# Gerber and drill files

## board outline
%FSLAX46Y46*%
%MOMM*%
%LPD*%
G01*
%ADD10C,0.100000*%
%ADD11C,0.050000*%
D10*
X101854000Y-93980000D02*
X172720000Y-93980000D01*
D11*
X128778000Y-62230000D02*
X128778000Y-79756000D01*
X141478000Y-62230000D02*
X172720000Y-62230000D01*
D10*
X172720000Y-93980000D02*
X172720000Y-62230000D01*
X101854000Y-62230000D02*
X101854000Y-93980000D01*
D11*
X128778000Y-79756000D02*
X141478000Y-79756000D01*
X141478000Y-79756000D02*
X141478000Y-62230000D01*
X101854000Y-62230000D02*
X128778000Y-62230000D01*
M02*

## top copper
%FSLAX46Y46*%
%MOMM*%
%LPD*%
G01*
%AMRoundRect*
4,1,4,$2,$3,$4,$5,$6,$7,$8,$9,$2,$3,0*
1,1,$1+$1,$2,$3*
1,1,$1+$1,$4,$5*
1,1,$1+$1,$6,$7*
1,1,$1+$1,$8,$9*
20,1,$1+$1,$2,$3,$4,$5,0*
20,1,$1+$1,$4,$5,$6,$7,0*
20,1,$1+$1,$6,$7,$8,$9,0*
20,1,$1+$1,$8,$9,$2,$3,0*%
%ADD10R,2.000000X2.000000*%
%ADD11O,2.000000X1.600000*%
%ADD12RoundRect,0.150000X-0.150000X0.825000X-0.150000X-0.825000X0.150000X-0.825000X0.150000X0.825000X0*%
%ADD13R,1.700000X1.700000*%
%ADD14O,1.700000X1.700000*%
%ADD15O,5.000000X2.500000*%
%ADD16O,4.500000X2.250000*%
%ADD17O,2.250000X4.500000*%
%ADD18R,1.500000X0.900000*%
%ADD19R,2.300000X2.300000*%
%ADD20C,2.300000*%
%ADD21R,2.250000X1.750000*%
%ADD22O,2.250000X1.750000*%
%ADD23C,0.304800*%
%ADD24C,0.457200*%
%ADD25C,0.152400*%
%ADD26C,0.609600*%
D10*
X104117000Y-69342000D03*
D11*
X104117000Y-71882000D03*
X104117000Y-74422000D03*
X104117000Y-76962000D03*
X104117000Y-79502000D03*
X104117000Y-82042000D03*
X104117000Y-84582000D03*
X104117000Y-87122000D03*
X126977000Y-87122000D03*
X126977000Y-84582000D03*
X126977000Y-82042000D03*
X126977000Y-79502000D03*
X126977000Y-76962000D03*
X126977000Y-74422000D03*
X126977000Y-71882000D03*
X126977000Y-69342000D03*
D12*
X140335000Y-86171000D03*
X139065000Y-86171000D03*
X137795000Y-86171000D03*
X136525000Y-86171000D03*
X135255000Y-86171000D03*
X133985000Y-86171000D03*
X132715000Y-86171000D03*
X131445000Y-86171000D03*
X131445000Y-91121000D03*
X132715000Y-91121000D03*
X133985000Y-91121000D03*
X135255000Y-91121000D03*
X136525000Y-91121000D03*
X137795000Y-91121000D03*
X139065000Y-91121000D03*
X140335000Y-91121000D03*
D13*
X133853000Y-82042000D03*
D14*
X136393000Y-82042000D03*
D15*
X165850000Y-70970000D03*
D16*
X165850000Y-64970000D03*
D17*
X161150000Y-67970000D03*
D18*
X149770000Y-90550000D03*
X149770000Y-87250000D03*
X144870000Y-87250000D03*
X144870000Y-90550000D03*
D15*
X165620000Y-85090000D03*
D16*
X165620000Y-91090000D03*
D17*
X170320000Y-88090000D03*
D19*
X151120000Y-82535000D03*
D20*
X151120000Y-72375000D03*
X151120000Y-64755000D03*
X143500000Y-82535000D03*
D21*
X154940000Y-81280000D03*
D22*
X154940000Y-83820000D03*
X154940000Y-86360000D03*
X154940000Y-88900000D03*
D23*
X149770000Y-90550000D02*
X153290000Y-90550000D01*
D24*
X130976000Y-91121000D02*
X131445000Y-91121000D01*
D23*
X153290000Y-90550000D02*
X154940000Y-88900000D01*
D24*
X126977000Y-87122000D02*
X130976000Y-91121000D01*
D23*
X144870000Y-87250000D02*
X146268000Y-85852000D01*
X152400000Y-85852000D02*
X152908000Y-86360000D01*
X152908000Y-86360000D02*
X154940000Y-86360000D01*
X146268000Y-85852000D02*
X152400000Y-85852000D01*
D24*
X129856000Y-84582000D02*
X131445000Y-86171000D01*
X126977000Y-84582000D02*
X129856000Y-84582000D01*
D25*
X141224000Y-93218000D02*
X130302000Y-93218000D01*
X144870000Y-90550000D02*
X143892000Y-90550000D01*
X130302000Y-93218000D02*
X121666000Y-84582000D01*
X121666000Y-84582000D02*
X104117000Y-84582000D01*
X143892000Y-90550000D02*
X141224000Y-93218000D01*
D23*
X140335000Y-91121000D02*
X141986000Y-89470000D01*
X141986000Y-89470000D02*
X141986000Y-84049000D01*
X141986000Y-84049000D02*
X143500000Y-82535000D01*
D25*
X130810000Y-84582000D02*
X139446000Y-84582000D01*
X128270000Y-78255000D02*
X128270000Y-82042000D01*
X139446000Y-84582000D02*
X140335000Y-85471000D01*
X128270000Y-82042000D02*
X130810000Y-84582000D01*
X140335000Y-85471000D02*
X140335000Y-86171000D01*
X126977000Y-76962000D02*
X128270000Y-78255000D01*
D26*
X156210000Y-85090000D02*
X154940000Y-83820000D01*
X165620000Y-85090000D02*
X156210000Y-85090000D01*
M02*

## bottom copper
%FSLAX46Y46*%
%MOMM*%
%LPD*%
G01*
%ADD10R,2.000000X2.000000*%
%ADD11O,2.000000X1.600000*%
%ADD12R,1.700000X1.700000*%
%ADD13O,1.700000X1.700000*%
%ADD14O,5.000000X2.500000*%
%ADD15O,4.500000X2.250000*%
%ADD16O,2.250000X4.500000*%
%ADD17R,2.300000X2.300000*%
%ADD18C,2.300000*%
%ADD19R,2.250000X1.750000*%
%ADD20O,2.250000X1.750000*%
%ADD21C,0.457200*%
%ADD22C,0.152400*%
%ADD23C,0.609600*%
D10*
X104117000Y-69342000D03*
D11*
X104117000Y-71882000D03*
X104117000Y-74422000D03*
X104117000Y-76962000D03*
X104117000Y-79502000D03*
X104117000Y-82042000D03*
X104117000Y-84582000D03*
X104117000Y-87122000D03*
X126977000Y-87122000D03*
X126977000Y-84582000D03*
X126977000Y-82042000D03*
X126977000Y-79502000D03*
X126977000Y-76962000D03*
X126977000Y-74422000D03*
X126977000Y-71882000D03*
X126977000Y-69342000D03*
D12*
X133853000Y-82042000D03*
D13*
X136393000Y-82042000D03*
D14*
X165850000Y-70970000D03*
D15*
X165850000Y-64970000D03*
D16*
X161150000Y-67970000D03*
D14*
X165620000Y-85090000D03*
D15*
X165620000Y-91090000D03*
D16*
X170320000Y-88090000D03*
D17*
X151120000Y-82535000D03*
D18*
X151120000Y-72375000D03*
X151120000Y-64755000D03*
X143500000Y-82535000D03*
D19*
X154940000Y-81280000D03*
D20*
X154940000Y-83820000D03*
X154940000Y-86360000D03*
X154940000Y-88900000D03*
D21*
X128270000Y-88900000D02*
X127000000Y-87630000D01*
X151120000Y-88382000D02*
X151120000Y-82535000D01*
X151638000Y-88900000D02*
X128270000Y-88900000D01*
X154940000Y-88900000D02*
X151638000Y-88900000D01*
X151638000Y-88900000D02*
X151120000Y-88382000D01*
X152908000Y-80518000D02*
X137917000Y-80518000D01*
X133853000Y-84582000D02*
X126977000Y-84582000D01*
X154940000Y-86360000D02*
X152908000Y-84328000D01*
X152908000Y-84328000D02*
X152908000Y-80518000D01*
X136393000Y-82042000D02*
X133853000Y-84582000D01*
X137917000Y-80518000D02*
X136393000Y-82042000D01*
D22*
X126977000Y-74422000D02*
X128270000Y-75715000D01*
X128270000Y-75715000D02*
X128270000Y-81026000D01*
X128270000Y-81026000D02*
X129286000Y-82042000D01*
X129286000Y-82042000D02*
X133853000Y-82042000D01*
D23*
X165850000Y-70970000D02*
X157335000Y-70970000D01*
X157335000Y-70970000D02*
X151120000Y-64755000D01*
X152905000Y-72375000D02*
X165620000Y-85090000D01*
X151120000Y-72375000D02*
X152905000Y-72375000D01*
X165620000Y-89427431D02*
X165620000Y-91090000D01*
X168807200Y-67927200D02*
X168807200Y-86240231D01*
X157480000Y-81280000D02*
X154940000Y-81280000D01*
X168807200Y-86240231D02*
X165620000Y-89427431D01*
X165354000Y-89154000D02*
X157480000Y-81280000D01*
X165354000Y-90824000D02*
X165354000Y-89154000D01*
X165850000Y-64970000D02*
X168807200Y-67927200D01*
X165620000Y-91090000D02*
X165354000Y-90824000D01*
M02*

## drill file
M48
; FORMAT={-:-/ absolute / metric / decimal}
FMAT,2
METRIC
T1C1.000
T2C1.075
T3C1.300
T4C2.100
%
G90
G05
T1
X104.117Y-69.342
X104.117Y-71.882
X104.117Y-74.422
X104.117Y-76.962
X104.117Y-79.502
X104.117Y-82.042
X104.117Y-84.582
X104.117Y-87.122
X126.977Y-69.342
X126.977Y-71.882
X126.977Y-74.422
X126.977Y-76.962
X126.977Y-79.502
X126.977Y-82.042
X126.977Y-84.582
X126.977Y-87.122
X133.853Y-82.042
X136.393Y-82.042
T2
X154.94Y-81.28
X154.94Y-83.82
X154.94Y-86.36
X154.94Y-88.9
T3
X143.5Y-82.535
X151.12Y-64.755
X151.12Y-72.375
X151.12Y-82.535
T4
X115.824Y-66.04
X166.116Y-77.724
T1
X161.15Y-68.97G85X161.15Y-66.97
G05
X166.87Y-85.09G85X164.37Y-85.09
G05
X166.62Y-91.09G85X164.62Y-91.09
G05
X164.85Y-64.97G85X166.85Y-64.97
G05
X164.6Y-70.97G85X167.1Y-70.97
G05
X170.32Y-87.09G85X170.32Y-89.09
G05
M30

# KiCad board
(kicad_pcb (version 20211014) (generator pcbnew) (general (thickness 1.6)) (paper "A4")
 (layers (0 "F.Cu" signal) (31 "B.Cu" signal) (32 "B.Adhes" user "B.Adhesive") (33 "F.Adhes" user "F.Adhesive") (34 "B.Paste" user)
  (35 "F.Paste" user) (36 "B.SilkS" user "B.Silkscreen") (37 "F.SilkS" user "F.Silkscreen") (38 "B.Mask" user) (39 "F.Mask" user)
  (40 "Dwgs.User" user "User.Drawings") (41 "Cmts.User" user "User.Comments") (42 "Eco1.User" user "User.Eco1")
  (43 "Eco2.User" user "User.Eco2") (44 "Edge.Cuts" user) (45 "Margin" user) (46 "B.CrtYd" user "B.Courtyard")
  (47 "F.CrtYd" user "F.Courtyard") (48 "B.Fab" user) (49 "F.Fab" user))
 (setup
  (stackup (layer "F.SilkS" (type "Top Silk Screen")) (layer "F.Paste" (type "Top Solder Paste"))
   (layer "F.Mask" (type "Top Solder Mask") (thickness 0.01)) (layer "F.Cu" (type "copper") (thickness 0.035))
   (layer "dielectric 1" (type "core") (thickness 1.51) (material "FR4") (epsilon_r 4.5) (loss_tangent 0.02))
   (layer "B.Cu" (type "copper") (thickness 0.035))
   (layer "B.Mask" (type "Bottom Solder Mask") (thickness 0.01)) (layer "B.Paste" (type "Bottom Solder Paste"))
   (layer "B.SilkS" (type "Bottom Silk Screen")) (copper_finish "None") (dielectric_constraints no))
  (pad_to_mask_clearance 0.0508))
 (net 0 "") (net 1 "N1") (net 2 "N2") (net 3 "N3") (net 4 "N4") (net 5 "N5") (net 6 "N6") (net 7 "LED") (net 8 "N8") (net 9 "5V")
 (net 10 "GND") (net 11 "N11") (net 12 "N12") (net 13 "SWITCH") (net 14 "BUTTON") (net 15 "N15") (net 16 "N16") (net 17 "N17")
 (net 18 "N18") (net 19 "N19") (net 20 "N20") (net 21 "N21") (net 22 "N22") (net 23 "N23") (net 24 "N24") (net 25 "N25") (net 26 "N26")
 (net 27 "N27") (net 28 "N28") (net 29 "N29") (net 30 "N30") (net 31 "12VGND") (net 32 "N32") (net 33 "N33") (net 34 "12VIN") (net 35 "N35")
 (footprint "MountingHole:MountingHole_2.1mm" (layer "F.Cu") (at 115.824 66.04)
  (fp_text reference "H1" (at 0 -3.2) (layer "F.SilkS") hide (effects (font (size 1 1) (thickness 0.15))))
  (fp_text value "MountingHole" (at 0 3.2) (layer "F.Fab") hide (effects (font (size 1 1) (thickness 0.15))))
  (pad "" np_thru_hole circle (at 0 0) (size 2.1 2.1) (drill 2.1) (layers *.Cu *.Mask)))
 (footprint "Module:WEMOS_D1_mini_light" (layer "F.Cu") (at 104.117 69.342)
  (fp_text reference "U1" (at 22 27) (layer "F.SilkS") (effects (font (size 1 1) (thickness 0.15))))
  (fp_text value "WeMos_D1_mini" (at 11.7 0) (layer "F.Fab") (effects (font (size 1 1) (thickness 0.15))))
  (pad "1" thru_hole rect (at 0 0) (size 2 2) (drill 1) (layers *.Cu *.Mask) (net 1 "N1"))
  (pad "2" thru_hole oval (at 0 2.54) (size 2 1.6) (drill 1) (layers *.Cu *.Mask) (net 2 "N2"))
  (pad "3" thru_hole oval (at 0 5.08) (size 2 1.6) (drill 1) (layers *.Cu *.Mask) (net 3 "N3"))
  (pad "4" thru_hole oval (at 0 7.62) (size 2 1.6) (drill 1) (layers *.Cu *.Mask) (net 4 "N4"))
  (pad "5" thru_hole oval (at 0 10.16) (size 2 1.6) (drill 1) (layers *.Cu *.Mask) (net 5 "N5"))
  (pad "6" thru_hole oval (at 0 12.7) (size 2 1.6) (drill 1) (layers *.Cu *.Mask) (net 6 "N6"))
  (pad "7" thru_hole oval (at 0 15.24) (size 2 1.6) (drill 1) (layers *.Cu *.Mask) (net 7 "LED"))
  (pad "8" thru_hole oval (at 0 17.78) (size 2 1.6) (drill 1) (layers *.Cu *.Mask) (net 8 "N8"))
  (pad "9" thru_hole oval (at 22.86 17.78) (size 2 1.6) (drill 1) (layers *.Cu *.Mask) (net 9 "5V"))
  (pad "10" thru_hole oval (at 22.86 15.24) (size 2 1.6) (drill 1) (layers *.Cu *.Mask) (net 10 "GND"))
  (pad "11" thru_hole oval (at 22.86 12.7) (size 2 1.6) (drill 1) (layers *.Cu *.Mask) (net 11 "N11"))
  (pad "12" thru_hole oval (at 22.86 10.16) (size 2 1.6) (drill 1) (layers *.Cu *.Mask) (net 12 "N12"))
  (pad "13" thru_hole oval (at 22.86 7.62) (size 2 1.6) (drill 1) (layers *.Cu *.Mask) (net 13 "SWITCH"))
  (pad "14" thru_hole oval (at 22.86 5.08) (size 2 1.6) (drill 1) (layers *.Cu *.Mask) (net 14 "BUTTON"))
  (pad "15" thru_hole oval (at 22.86 2.54) (size 2 1.6) (drill 1) (layers *.Cu *.Mask) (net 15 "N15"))
  (pad "16" thru_hole oval (at 22.86 0) (size 2 1.6) (drill 1) (layers *.Cu *.Mask) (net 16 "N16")))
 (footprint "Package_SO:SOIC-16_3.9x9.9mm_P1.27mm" (layer "F.Cu") (at 135.89 88.646 -90)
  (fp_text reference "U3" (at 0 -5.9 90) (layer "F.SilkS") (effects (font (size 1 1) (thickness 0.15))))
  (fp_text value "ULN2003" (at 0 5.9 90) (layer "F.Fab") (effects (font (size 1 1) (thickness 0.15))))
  (pad "1" smd roundrect (at -2.475 -4.445 270) (size 1.95 0.6) (layers "F.Cu" "F.Paste" "F.Mask") (roundrect_rratio 0.25) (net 13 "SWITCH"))
  (pad "2" smd roundrect (at -2.475 -3.175 270) (size 1.95 0.6) (layers "F.Cu" "F.Paste" "F.Mask") (roundrect_rratio 0.25) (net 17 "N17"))
  (pad "3" smd roundrect (at -2.475 -1.905 270) (size 1.95 0.6) (layers "F.Cu" "F.Paste" "F.Mask") (roundrect_rratio 0.25) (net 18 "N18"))
  (pad "4" smd roundrect (at -2.475 -0.635 270) (size 1.95 0.6) (layers "F.Cu" "F.Paste" "F.Mask") (roundrect_rratio 0.25) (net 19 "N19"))
  (pad "5" smd roundrect (at -2.475 0.635 270) (size 1.95 0.6) (layers "F.Cu" "F.Paste" "F.Mask") (roundrect_rratio 0.25) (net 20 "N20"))
  (pad "6" smd roundrect (at -2.475 1.905 270) (size 1.95 0.6) (layers "F.Cu" "F.Paste" "F.Mask") (roundrect_rratio 0.25) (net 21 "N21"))
  (pad "7" smd roundrect (at -2.475 3.175 270) (size 1.95 0.6) (layers "F.Cu" "F.Paste" "F.Mask") (roundrect_rratio 0.25) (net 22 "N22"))
  (pad "8" smd roundrect (at -2.475 4.445 270) (size 1.95 0.6) (layers "F.Cu" "F.Paste" "F.Mask") (roundrect_rratio 0.25) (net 10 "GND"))
  (pad "9" smd roundrect (at 2.475 4.445 270) (size 1.95 0.6) (layers "F.Cu" "F.Paste" "F.Mask") (roundrect_rratio 0.25) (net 9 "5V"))
  (pad "10" smd roundrect (at 2.475 3.175 270) (size 1.95 0.6) (layers "F.Cu" "F.Paste" "F.Mask") (roundrect_rratio 0.25) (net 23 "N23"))
  (pad "11" smd roundrect (at 2.475 1.905 270) (size 1.95 0.6) (layers "F.Cu" "F.Paste" "F.Mask") (roundrect_rratio 0.25) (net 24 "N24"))
  (pad "12" smd roundrect (at 2.475 0.635 270) (size 1.95 0.6) (layers "F.Cu" "F.Paste" "F.Mask") (roundrect_rratio 0.25) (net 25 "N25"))
  (pad "13" smd roundrect (at 2.475 -0.635 270) (size 1.95 0.6) (layers "F.Cu" "F.Paste" "F.Mask") (roundrect_rratio 0.25) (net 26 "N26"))
  (pad "14" smd roundrect (at 2.475 -1.905 270) (size 1.95 0.6) (layers "F.Cu" "F.Paste" "F.Mask") (roundrect_rratio 0.25) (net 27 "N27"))
  (pad "15" smd roundrect (at 2.475 -3.175 270) (size 1.95 0.6) (layers "F.Cu" "F.Paste" "F.Mask") (roundrect_rratio 0.25) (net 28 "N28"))
  (pad "16" smd roundrect (at 2.475 -4.445 270) (size 1.95 0.6) (layers "F.Cu" "F.Paste" "F.Mask") (roundrect_rratio 0.25) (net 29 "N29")))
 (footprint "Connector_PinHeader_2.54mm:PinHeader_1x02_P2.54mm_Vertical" (layer "F.Cu") (at 133.853 82.042 90)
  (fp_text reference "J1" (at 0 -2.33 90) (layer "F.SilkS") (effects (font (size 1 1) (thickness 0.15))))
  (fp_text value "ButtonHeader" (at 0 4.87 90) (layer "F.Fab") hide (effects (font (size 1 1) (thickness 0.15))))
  (pad "1" thru_hole rect (at 0 0 90) (size 1.7 1.7) (drill 1) (layers *.Cu *.Mask) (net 14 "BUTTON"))
  (pad "2" thru_hole oval (at 0 2.54 90) (size 1.7 1.7) (drill 1) (layers *.Cu *.Mask) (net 10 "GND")))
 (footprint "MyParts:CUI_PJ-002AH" (layer "F.Cu") (at 165.85 70.97 90)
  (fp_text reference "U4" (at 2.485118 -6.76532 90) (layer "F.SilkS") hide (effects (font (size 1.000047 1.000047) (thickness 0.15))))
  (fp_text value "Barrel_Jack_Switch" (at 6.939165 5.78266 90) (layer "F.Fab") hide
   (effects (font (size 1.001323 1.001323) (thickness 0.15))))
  (pad "1" thru_hole oval locked (at 0 0 90) (size 2.5 5) (drill oval 1 3.5) (layers *.Cu *.Mask) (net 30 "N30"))
  (pad "2" thru_hole oval locked (at 6 0 90) (size 2.25 4.5) (drill oval 1 3) (layers *.Cu *.Mask) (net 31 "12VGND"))
  (pad "3" thru_hole oval locked (at 3 -4.7 90) (size 4.5 2.25) (drill oval 3 1) (layers *.Cu *.Mask) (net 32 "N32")))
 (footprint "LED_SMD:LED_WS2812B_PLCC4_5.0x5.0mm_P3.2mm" (layer "F.Cu") (at 147.32 88.9 180)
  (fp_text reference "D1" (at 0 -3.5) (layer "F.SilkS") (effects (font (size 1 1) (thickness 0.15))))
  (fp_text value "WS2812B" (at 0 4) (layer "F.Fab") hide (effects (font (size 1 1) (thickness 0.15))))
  (pad "1" smd rect (at -2.45 -1.65 180) (size 1.5 0.9) (layers "F.Cu" "F.Paste" "F.Mask") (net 9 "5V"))
  (pad "2" smd rect (at -2.45 1.65 180) (size 1.5 0.9) (layers "F.Cu" "F.Paste" "F.Mask") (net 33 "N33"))
  (pad "3" smd rect (at 2.45 1.65 180) (size 1.5 0.9) (layers "F.Cu" "F.Paste" "F.Mask") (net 10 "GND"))
  (pad "4" smd rect (at 2.45 -1.65 180) (size 1.5 0.9) (layers "F.Cu" "F.Paste" "F.Mask") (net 7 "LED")))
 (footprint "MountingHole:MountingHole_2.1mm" (layer "F.Cu") (at 166.116 77.724)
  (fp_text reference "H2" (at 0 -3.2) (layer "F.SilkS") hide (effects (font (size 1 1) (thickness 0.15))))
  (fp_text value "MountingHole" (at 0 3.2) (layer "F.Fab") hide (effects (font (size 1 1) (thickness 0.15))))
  (pad "" np_thru_hole circle (at 0 0) (size 2.1 2.1) (drill 2.1) (layers *.Cu *.Mask)))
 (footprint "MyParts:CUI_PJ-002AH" (layer "F.Cu") (at 165.62 85.09 -90)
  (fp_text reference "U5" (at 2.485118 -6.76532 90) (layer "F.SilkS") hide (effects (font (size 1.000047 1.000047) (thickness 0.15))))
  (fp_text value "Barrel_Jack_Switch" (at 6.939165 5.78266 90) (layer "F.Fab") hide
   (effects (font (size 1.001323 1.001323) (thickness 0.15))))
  (pad "1" thru_hole oval locked (at 0 0 270) (size 2.5 5) (drill oval 1 3.5) (layers *.Cu *.Mask) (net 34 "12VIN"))
  (pad "2" thru_hole oval locked (at 6 0 270) (size 2.25 4.5) (drill oval 1 3) (layers *.Cu *.Mask) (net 31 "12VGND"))
  (pad "3" thru_hole oval locked (at 3 -4.7 270) (size 4.5 2.25) (drill oval 3 1) (layers *.Cu *.Mask) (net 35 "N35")))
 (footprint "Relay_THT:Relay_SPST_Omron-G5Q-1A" (layer "F.Cu") (at 151.12 82.535 90)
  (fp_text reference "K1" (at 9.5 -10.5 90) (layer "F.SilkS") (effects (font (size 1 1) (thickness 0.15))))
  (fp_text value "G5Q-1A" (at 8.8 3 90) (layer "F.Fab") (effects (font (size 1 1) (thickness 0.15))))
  (pad "1" thru_hole rect (at 0 0 270) (size 2.3 2.3) (drill 1.3) (layers *.Cu *.Mask) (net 9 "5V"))
  (pad "2" thru_hole circle (at 10.16 0 270) (size 2.3 2.3) (drill 1.3) (layers *.Cu *.Mask) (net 34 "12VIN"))
  (pad "3" thru_hole circle (at 17.78 0 270) (size 2.3 2.3) (drill 1.3) (layers *.Cu *.Mask) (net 30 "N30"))
  (pad "5" thru_hole circle (at 0 -7.62 270) (size 2.3 2.3) (drill 1.3) (layers *.Cu *.Mask) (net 29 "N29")))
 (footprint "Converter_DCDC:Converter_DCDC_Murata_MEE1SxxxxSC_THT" (layer "F.Cu") (at 154.94 81.28)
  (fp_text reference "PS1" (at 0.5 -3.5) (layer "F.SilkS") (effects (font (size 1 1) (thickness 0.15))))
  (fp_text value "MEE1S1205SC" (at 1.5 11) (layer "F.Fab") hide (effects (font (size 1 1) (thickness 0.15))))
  (pad "1" thru_hole rect (at 0 0 270) (size 1.75 2.25) (drill 1.075) (layers *.Cu *.Mask) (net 31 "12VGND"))
  (pad "2" thru_hole oval (at 0 2.54 270) (size 1.75 2.25) (drill 1.075) (layers *.Cu *.Mask) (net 34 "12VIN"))
  (pad "3" thru_hole oval (at 0 5.08 270) (size 1.75 2.25) (drill 1.075) (layers *.Cu *.Mask) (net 10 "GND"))
  (pad "4" thru_hole oval (at 0 7.62 270) (size 1.75 2.25) (drill 1.075) (layers *.Cu *.Mask) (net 9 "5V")))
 (gr_line (start 101.854 93.98) (end 172.72 93.98) (layer "Edge.Cuts") (width 0.1))
 (gr_line (start 128.778 62.23) (end 128.778 79.756) (layer "Edge.Cuts") (width 0.05))
 (gr_line (start 141.478 62.23) (end 172.72 62.23) (layer "Edge.Cuts") (width 0.05))
 (gr_line (start 172.72 93.98) (end 172.72 62.23) (layer "Edge.Cuts") (width 0.1))
 (gr_line (start 101.854 62.23) (end 101.854 93.98) (layer "Edge.Cuts") (width 0.1))
 (gr_line (start 128.778 79.756) (end 141.478 79.756) (layer "Edge.Cuts") (width 0.05))
 (gr_line (start 141.478 79.756) (end 141.478 62.23) (layer "Edge.Cuts") (width 0.05))
 (gr_line (start 101.854 62.23) (end 128.778 62.23) (layer "Edge.Cuts") (width 0.05))
 (segment (start 149.77 90.55) (end 153.29 90.55) (width 0.3048) (layer "F.Cu") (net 9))
 (segment (start 130.976 91.121) (end 131.445 91.121) (width 0.4572) (layer "F.Cu") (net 9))
 (segment (start 153.29 90.55) (end 154.94 88.9) (width 0.3048) (layer "F.Cu") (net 9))
 (segment (start 126.977 87.122) (end 130.976 91.121) (width 0.4572) (layer "F.Cu") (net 9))
 (segment (start 128.27 88.9) (end 127 87.63) (width 0.4572) (layer "B.Cu") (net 9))
 (segment (start 151.12 88.382) (end 151.12 82.535) (width 0.4572) (layer "B.Cu") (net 9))
 (segment (start 151.638 88.9) (end 128.27 88.9) (width 0.4572) (layer "B.Cu") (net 9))
 (segment (start 154.94 88.9) (end 151.638 88.9) (width 0.4572) (layer "B.Cu") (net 9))
 (segment (start 151.638 88.9) (end 151.12 88.382) (width 0.4572) (layer "B.Cu") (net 9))
 (segment (start 144.87 87.25) (end 146.268 85.852) (width 0.3048) (layer "F.Cu") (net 10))
 (segment (start 152.4 85.852) (end 152.908 86.36) (width 0.3048) (layer "F.Cu") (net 10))
 (segment (start 152.908 86.36) (end 154.94 86.36) (width 0.3048) (layer "F.Cu") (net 10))
 (segment (start 146.268 85.852) (end 152.4 85.852) (width 0.3048) (layer "F.Cu") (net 10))
 (segment (start 129.856 84.582) (end 131.445 86.171) (width 0.4572) (layer "F.Cu") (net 10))
 (segment (start 126.977 84.582) (end 129.856 84.582) (width 0.4572) (layer "F.Cu") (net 10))
 (segment (start 152.908 80.518) (end 137.917 80.518) (width 0.4572) (layer "B.Cu") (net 10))
 (segment (start 133.853 84.582) (end 126.977 84.582) (width 0.4572) (layer "B.Cu") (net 10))
 (segment (start 154.94 86.36) (end 152.908 84.328) (width 0.4572) (layer "B.Cu") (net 10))
 (segment (start 152.908 84.328) (end 152.908 80.518) (width 0.4572) (layer "B.Cu") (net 10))
 (segment (start 136.393 82.042) (end 133.853 84.582) (width 0.4572) (layer "B.Cu") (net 10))
 (segment (start 137.917 80.518) (end 136.393 82.042) (width 0.4572) (layer "B.Cu") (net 10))
 (segment (start 141.224 93.218) (end 130.302 93.218) (width 0.1524) (layer "F.Cu") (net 7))
 (segment (start 144.87 90.55) (end 143.892 90.55) (width 0.1524) (layer "F.Cu") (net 7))
 (segment (start 130.302 93.218) (end 121.666 84.582) (width 0.1524) (layer "F.Cu") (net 7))
 (segment (start 121.666 84.582) (end 104.117 84.582) (width 0.1524) (layer "F.Cu") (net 7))
 (segment (start 143.892 90.55) (end 141.224 93.218) (width 0.1524) (layer "F.Cu") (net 7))
 (segment (start 126.977 74.422) (end 128.27 75.715) (width 0.1524) (layer "B.Cu") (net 14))
 (segment (start 128.27 75.715) (end 128.27 81.026) (width 0.1524) (layer "B.Cu") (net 14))
 (segment (start 128.27 81.026) (end 129.286 82.042) (width 0.1524) (layer "B.Cu") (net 14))
 (segment (start 129.286 82.042) (end 133.853 82.042) (width 0.1524) (layer "B.Cu") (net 14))
 (segment (start 165.85 70.97) (end 157.335 70.97) (width 0.6096) (layer "B.Cu") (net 30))
 (segment (start 157.335 70.97) (end 151.12 64.755) (width 0.6096) (layer "B.Cu") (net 30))
 (segment (start 140.335 91.121) (end 141.986 89.47) (width 0.3048) (layer "F.Cu") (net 29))
 (segment (start 141.986 89.47) (end 141.986 84.049) (width 0.3048) (layer "F.Cu") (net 29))
 (segment (start 141.986 84.049) (end 143.5 82.535) (width 0.3048) (layer "F.Cu") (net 29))
 (segment (start 130.81 84.582) (end 139.446 84.582) (width 0.1524) (layer "F.Cu") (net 13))
 (segment (start 128.27 78.255) (end 128.27 82.042) (width 0.1524) (layer "F.Cu") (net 13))
 (segment (start 139.446 84.582) (end 140.335 85.471) (width 0.1524) (layer "F.Cu") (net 13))
 (segment (start 128.27 82.042) (end 130.81 84.582) (width 0.1524) (layer "F.Cu") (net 13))
 (segment (start 140.335 85.471) (end 140.335 86.171) (width 0.1524) (layer "F.Cu") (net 13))
 (segment (start 126.977 76.962) (end 128.27 78.255) (width 0.1524) (layer "F.Cu") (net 13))
 (segment (start 156.21 85.09) (end 154.94 83.82) (width 0.6096) (layer "F.Cu") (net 34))
 (segment (start 165.62 85.09) (end 156.21 85.09) (width 0.6096) (layer "F.Cu") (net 34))
 (segment (start 152.905 72.375) (end 165.62 85.09) (width 0.6096) (layer "B.Cu") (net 34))
 (segment (start 151.12 72.375) (end 152.905 72.375) (width 0.6096) (layer "B.Cu") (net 34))
 (segment (start 165.62 89.427431) (end 165.62 91.09) (width 0.6096) (layer "B.Cu") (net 31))
 (segment (start 168.8072 67.9272) (end 168.8072 86.240231) (width 0.6096) (layer "B.Cu") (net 31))
 (segment (start 157.48 81.28) (end 154.94 81.28) (width 0.6096) (layer "B.Cu") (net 31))
 (segment (start 168.8072 86.240231) (end 165.62 89.427431) (width 0.6096) (layer "B.Cu") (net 31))
 (segment (start 165.354 89.154) (end 157.48 81.28) (width 0.6096) (layer "B.Cu") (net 31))
 (segment (start 165.354 90.824) (end 165.354 89.154) (width 0.6096) (layer "B.Cu") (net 31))
 (segment (start 165.85 64.97) (end 168.8072 67.9272) (width 0.6096) (layer "B.Cu") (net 31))
 (segment (start 165.62 91.09) (end 165.354 90.824) (width 0.6096) (layer "B.Cu") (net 31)))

